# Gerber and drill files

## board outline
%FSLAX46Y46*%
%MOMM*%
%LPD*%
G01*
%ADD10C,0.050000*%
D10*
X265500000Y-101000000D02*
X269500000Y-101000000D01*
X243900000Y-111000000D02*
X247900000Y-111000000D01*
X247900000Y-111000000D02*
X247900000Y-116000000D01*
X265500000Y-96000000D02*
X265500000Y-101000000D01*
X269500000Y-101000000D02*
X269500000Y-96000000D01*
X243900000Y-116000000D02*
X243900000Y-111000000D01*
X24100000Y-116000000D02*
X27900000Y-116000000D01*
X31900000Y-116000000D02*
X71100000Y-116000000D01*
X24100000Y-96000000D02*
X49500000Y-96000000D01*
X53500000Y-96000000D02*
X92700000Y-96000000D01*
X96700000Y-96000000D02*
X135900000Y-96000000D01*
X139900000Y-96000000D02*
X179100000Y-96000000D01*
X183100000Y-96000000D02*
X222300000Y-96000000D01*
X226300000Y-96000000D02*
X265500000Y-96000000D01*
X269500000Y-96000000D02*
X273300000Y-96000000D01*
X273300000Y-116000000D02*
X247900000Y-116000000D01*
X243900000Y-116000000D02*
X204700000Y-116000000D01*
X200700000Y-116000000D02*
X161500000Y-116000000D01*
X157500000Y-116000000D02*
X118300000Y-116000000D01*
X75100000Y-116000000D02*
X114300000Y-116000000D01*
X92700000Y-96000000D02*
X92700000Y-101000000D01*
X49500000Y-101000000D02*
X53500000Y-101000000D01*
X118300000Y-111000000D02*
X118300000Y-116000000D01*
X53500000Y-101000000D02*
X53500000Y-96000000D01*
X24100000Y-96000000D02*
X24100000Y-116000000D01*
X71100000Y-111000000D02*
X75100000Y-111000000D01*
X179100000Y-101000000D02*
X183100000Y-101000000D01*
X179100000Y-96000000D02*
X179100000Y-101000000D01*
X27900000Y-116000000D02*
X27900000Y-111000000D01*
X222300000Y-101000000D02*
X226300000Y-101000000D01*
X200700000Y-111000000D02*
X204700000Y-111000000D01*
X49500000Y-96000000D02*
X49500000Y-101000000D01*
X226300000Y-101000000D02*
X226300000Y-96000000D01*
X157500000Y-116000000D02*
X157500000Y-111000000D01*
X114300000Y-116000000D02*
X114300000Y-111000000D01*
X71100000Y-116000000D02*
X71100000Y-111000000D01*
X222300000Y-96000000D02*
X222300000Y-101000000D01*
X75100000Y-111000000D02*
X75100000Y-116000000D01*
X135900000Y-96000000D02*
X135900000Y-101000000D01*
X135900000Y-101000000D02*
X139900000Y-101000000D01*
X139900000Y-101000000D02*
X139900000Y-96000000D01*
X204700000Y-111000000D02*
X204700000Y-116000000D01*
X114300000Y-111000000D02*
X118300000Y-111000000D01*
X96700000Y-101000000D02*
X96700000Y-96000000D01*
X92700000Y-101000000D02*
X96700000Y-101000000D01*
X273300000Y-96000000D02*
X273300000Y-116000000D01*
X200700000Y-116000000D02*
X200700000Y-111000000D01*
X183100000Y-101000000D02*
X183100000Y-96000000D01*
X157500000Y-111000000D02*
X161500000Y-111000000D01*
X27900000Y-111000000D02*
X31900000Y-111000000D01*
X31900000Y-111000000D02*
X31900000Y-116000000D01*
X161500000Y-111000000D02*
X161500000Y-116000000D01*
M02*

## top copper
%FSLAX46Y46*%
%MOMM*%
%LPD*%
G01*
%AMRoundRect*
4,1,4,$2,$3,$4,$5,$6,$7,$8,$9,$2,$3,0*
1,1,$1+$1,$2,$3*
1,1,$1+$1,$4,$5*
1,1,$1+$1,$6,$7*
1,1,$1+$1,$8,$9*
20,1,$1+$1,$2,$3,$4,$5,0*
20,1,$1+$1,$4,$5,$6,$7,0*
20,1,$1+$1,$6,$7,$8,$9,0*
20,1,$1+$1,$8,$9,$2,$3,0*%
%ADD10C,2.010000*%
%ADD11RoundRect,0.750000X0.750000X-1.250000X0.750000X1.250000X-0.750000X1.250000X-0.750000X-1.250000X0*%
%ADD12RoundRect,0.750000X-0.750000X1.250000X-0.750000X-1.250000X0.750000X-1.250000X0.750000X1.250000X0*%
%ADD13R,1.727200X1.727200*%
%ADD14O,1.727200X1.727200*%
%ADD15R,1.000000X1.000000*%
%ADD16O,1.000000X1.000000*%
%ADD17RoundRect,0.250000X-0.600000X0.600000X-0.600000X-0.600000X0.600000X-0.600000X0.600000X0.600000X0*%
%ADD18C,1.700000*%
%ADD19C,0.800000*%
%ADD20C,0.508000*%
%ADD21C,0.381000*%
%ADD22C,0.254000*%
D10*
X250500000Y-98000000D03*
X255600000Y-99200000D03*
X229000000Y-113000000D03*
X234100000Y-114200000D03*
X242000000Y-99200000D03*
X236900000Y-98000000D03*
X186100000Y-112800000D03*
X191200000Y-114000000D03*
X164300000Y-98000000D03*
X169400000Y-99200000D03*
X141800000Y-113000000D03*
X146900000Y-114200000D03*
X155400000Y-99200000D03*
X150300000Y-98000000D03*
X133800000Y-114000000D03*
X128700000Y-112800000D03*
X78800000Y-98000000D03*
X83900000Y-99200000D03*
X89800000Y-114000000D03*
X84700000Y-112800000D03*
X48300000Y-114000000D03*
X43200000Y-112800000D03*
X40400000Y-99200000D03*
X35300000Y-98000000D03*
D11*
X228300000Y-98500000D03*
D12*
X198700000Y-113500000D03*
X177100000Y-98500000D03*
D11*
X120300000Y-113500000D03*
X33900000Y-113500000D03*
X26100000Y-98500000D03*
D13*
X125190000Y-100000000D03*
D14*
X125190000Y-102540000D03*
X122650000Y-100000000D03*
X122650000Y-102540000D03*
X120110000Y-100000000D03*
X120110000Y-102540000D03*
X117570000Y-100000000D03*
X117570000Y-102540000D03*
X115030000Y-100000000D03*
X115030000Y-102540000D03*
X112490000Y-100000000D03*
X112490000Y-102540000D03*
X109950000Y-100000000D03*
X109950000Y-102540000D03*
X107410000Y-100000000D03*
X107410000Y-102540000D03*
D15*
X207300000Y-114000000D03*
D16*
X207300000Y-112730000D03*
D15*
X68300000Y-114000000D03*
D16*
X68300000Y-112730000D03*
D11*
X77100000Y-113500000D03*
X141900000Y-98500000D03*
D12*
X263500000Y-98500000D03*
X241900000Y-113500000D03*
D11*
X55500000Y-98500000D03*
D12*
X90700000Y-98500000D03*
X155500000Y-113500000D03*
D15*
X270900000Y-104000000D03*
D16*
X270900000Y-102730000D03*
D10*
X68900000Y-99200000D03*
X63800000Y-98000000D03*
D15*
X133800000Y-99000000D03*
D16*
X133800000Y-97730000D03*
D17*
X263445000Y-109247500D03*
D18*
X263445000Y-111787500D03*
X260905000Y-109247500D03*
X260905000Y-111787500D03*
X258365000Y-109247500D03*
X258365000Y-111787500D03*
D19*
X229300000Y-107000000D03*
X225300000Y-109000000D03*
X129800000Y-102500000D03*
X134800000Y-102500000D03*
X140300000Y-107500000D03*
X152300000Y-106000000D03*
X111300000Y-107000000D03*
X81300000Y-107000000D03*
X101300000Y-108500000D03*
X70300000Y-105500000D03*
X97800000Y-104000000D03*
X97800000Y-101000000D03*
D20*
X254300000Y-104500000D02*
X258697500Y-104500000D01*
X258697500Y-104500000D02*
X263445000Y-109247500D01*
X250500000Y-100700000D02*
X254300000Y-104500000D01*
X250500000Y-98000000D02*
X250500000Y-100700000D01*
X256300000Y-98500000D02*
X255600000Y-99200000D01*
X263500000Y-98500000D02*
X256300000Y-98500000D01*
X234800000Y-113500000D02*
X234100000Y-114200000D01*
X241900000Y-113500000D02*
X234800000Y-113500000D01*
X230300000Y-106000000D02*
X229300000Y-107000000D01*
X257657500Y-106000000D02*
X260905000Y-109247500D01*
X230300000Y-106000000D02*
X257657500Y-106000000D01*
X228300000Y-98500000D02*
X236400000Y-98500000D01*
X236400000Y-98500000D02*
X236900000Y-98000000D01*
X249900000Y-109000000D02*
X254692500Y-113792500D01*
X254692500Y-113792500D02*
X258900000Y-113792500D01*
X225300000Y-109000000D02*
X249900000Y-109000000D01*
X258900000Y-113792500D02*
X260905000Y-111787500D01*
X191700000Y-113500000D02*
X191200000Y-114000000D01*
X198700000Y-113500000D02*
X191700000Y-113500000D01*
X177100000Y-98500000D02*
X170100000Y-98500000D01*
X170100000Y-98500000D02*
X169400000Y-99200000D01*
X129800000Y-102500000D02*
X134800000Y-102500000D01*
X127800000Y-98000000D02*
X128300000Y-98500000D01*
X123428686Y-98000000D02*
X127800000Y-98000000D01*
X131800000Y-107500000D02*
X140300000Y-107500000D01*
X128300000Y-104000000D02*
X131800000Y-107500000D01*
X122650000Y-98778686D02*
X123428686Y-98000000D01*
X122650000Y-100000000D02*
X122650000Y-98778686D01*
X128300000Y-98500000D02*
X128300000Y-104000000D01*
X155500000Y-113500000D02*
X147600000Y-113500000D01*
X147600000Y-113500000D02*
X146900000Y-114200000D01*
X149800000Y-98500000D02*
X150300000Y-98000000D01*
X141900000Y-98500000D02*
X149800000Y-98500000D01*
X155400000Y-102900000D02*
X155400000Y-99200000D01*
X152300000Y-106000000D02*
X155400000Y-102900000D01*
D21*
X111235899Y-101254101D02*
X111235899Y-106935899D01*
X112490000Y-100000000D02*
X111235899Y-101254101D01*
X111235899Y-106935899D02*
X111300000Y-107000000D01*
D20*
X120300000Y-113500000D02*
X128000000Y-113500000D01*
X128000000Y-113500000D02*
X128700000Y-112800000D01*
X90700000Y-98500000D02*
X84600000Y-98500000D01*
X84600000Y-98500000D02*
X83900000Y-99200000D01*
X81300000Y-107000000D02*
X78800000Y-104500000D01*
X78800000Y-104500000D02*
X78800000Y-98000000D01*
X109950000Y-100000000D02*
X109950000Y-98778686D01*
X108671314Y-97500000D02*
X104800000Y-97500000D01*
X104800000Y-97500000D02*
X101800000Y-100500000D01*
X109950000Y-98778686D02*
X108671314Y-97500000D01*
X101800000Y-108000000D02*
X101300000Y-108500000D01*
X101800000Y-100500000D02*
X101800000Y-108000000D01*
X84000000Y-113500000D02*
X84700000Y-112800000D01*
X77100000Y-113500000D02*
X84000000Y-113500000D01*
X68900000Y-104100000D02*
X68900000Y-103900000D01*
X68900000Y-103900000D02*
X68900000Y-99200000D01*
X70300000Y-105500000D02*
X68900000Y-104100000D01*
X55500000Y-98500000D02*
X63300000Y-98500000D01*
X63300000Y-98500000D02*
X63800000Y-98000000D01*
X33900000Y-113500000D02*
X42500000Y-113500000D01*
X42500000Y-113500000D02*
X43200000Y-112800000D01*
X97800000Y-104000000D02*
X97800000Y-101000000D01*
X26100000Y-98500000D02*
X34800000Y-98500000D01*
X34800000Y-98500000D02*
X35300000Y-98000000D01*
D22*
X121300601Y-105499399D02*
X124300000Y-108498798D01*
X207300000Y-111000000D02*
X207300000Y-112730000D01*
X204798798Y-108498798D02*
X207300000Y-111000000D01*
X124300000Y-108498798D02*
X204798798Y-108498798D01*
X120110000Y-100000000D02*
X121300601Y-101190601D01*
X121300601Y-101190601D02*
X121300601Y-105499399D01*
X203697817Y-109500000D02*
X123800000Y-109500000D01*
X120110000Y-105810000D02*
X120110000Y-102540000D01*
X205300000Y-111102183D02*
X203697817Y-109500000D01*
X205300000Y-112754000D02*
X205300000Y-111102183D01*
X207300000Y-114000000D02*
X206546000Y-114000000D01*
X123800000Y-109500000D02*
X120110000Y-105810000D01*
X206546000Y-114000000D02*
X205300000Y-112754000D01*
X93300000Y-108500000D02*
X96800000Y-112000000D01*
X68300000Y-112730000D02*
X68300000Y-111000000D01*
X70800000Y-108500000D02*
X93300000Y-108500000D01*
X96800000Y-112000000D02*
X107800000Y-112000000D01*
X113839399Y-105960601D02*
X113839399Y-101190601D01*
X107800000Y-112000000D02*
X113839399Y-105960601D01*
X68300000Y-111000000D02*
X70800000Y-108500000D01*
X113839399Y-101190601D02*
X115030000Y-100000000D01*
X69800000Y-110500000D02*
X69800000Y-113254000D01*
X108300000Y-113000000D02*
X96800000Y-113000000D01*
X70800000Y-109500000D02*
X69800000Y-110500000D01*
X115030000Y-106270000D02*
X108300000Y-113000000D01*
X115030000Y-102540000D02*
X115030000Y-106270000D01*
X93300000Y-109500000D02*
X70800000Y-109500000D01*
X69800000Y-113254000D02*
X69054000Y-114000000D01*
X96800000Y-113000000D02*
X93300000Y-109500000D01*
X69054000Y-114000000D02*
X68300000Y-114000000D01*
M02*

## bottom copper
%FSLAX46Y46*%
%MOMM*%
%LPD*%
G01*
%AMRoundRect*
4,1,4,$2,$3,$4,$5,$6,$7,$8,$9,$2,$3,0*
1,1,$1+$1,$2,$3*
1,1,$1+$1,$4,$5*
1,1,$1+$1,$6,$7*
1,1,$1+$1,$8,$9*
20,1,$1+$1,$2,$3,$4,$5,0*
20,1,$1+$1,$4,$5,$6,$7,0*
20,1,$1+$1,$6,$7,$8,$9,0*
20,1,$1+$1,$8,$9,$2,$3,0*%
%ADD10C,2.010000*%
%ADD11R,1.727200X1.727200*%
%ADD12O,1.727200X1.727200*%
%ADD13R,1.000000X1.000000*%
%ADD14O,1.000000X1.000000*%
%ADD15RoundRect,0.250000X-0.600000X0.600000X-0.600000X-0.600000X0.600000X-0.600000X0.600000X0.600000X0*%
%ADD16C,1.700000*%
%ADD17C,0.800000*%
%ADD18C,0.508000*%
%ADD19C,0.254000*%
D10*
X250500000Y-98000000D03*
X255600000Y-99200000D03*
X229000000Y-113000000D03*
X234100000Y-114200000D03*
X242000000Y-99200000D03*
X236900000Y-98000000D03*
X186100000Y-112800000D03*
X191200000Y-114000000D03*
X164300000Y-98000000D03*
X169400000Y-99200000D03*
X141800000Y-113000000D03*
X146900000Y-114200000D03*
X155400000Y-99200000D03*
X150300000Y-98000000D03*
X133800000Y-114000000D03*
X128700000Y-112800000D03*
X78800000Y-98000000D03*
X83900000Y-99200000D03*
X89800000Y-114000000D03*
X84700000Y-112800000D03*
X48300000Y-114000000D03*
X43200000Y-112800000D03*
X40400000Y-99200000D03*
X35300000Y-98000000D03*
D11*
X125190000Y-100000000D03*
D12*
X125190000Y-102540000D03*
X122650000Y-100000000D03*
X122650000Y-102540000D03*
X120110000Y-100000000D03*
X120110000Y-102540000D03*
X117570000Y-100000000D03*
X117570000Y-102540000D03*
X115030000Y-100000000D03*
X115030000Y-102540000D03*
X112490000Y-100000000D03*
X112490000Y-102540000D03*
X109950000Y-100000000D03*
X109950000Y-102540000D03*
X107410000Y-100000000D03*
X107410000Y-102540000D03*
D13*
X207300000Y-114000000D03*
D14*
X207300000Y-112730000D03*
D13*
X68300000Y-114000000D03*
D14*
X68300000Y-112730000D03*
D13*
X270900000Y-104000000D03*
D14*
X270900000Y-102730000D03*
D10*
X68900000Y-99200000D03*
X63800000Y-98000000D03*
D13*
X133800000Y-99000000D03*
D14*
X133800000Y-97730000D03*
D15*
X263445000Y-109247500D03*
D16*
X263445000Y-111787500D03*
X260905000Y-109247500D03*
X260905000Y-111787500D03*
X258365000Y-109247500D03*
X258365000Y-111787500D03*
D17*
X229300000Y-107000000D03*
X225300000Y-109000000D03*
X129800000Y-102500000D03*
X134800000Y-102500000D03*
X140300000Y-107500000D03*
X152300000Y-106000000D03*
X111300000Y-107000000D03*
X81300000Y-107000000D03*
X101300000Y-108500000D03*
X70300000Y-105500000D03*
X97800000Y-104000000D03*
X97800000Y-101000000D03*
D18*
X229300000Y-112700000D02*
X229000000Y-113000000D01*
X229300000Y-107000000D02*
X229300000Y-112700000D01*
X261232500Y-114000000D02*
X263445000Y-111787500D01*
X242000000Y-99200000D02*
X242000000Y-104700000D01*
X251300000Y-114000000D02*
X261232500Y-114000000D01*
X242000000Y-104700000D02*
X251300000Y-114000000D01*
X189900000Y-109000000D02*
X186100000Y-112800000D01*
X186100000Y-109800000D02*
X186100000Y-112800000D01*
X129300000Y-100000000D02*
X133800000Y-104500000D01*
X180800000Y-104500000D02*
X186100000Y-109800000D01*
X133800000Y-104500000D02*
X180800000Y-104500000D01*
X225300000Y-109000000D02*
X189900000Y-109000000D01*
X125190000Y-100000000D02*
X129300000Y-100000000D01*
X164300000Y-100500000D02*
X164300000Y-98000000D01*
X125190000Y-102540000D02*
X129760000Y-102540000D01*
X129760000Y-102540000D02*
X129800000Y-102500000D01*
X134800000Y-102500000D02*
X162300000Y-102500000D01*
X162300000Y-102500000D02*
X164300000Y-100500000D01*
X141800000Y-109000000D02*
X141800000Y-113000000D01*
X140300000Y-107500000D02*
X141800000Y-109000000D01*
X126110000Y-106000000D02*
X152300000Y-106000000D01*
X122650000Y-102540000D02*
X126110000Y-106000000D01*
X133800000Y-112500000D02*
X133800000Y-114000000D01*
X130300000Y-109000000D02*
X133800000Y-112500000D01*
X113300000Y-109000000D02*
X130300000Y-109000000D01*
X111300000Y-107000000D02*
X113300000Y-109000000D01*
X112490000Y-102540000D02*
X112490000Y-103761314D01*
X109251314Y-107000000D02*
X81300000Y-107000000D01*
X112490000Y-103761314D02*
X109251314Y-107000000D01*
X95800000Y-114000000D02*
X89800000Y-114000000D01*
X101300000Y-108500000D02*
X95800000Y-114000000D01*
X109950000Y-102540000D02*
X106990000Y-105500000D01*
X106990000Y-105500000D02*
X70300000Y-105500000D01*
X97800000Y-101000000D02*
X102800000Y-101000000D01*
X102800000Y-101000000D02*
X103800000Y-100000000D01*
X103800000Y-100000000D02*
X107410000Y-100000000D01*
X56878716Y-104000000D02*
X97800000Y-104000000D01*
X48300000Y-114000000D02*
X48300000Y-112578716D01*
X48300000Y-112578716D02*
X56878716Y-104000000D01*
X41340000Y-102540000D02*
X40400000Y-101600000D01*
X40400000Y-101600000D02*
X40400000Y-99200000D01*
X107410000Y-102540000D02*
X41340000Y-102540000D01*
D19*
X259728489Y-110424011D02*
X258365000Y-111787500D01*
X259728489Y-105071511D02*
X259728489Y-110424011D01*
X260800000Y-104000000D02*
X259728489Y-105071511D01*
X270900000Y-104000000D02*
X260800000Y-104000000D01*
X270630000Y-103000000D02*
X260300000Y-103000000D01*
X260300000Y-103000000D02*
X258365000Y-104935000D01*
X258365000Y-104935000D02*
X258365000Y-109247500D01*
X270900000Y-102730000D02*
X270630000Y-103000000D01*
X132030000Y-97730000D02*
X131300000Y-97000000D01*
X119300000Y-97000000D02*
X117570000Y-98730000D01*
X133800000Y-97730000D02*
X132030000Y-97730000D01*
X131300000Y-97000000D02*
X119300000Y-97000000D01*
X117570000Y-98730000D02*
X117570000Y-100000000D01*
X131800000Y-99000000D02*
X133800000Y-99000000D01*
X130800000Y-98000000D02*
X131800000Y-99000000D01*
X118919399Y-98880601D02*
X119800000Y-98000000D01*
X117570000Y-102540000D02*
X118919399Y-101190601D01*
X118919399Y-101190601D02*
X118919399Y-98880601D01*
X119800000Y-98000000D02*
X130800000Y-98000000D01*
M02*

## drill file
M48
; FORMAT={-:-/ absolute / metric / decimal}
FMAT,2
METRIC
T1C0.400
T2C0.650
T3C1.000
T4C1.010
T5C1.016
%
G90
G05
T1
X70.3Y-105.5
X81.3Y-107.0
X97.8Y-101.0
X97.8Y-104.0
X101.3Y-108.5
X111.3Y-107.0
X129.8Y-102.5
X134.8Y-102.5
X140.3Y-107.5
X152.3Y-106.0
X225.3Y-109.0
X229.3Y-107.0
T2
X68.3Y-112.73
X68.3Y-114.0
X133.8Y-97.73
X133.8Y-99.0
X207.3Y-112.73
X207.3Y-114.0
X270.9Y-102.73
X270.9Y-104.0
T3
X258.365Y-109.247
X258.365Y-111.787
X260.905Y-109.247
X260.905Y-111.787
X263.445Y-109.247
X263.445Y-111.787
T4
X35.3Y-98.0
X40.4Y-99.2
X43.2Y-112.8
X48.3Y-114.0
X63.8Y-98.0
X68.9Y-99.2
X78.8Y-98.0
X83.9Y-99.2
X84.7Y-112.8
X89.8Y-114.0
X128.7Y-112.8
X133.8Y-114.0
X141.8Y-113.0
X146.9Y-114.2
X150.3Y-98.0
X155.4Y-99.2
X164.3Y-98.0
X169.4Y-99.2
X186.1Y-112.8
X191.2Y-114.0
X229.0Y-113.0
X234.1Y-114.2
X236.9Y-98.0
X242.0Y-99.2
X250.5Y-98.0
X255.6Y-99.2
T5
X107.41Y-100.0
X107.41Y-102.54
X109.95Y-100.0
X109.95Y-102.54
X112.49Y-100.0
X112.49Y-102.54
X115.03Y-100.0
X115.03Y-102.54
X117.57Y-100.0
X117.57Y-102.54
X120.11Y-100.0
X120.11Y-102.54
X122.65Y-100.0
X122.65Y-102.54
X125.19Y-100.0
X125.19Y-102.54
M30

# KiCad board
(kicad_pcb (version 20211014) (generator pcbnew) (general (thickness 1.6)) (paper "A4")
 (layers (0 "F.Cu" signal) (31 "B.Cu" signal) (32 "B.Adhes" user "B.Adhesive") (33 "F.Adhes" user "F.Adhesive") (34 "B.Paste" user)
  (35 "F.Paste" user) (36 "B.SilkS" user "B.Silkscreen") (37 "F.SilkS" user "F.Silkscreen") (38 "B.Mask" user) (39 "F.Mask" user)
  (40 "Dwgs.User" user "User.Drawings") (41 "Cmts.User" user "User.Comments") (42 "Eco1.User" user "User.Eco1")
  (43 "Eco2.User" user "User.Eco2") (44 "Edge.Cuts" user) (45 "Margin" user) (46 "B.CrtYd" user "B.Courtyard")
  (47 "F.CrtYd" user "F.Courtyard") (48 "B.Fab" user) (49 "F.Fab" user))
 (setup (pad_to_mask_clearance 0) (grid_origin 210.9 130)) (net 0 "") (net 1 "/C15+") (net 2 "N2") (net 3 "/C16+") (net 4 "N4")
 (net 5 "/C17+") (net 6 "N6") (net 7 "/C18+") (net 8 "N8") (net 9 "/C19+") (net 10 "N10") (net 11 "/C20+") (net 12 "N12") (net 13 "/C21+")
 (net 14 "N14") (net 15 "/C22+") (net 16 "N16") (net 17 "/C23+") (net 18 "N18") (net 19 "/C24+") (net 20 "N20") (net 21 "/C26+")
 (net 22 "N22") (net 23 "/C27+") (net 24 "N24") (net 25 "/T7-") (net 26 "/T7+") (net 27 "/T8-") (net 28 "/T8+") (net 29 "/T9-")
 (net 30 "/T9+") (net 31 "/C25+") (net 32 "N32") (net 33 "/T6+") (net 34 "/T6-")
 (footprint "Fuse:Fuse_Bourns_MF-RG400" (layer "F.Cu") (at 250.5 98)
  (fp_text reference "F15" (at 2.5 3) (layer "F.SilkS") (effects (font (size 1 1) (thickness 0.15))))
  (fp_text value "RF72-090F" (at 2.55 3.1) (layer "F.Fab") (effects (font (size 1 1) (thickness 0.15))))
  (pad "1" thru_hole circle locked (at 0 0) (size 2.01 2.01) (drill 1.01) (layers *.Cu *.Mask) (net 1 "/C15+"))
  (pad "2" thru_hole circle locked (at 5.1 1.2) (size 2.01 2.01) (drill 1.01) (layers *.Cu *.Mask) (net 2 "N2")))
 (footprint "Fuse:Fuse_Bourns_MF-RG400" (layer "F.Cu") (at 229 113)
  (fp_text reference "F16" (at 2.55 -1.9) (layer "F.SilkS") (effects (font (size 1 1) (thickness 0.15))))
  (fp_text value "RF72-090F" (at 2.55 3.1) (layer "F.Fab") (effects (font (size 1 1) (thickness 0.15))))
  (pad "1" thru_hole circle locked (at 0 0) (size 2.01 2.01) (drill 1.01) (layers *.Cu *.Mask) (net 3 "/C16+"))
  (pad "2" thru_hole circle locked (at 5.1 1.2) (size 2.01 2.01) (drill 1.01) (layers *.Cu *.Mask) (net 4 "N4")))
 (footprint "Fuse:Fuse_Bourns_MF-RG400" (layer "F.Cu") (at 242 99.2 180)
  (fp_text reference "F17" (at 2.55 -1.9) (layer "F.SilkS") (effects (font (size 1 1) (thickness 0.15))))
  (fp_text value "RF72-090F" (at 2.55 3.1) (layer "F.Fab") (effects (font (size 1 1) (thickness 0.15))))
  (pad "1" thru_hole circle locked (at 0 0 180) (size 2.01 2.01) (drill 1.01) (layers *.Cu *.Mask) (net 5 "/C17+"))
  (pad "2" thru_hole circle locked (at 5.1 1.2 180) (size 2.01 2.01) (drill 1.01) (layers *.Cu *.Mask) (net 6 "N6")))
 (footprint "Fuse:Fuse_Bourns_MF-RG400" (layer "F.Cu") (at 186.1 112.8)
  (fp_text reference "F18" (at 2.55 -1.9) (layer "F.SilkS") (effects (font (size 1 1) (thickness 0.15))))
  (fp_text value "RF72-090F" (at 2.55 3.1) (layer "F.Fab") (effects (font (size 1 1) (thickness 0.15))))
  (pad "1" thru_hole circle locked (at 0 0) (size 2.01 2.01) (drill 1.01) (layers *.Cu *.Mask) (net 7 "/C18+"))
  (pad "2" thru_hole circle locked (at 5.1 1.2) (size 2.01 2.01) (drill 1.01) (layers *.Cu *.Mask) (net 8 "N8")))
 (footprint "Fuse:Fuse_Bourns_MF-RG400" (layer "F.Cu") (at 164.3 98)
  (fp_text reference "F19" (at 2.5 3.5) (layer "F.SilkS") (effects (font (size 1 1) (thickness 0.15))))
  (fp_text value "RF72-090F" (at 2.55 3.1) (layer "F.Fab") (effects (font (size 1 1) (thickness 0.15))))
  (pad "1" thru_hole circle locked (at 0 0) (size 2.01 2.01) (drill 1.01) (layers *.Cu *.Mask) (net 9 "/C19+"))
  (pad "2" thru_hole circle locked (at 5.1 1.2) (size 2.01 2.01) (drill 1.01) (layers *.Cu *.Mask) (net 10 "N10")))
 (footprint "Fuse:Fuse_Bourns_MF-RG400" (layer "F.Cu") (at 141.8 113)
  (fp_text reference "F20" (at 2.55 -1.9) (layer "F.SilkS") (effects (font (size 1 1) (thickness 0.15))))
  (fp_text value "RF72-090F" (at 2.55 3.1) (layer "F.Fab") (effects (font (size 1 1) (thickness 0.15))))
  (pad "1" thru_hole circle locked (at 0 0) (size 2.01 2.01) (drill 1.01) (layers *.Cu *.Mask) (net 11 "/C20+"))
  (pad "2" thru_hole circle locked (at 5.1 1.2) (size 2.01 2.01) (drill 1.01) (layers *.Cu *.Mask) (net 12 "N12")))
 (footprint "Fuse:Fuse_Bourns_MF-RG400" (layer "F.Cu") (at 155.4 99.2 180)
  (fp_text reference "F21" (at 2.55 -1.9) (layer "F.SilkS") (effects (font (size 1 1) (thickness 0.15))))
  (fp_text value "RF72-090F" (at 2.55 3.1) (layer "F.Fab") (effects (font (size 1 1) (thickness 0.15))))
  (pad "1" thru_hole circle locked (at 0 0 180) (size 2.01 2.01) (drill 1.01) (layers *.Cu *.Mask) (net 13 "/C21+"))
  (pad "2" thru_hole circle locked (at 5.1 1.2 180) (size 2.01 2.01) (drill 1.01) (layers *.Cu *.Mask) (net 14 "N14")))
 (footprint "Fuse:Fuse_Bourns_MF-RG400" (layer "F.Cu") (at 133.8 114 180)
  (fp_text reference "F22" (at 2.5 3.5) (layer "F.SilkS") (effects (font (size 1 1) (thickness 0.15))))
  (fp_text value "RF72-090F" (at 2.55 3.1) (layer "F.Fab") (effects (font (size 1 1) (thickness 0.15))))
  (pad "1" thru_hole circle locked (at 0 0 180) (size 2.01 2.01) (drill 1.01) (layers *.Cu *.Mask) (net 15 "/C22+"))
  (pad "2" thru_hole circle locked (at 5.1 1.2 180) (size 2.01 2.01) (drill 1.01) (layers *.Cu *.Mask) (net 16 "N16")))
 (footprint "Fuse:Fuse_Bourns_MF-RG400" (layer "F.Cu") (at 78.8 98)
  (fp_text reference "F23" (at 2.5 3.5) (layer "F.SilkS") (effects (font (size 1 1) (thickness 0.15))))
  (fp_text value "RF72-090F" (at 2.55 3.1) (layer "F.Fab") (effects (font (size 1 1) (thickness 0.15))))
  (pad "1" thru_hole circle locked (at 0 0) (size 2.01 2.01) (drill 1.01) (layers *.Cu *.Mask) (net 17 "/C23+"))
  (pad "2" thru_hole circle locked (at 5.1 1.2) (size 2.01 2.01) (drill 1.01) (layers *.Cu *.Mask) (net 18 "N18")))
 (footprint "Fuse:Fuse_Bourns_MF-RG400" (layer "F.Cu") (at 89.8 114 180)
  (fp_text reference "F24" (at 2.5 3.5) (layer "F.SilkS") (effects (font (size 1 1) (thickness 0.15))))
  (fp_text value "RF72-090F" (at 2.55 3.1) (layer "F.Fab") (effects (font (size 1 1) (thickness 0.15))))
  (pad "1" thru_hole circle locked (at 0 0 180) (size 2.01 2.01) (drill 1.01) (layers *.Cu *.Mask) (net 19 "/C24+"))
  (pad "2" thru_hole circle locked (at 5.1 1.2 180) (size 2.01 2.01) (drill 1.01) (layers *.Cu *.Mask) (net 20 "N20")))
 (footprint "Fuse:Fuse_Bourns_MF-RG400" (layer "F.Cu") (at 48.3 114 180)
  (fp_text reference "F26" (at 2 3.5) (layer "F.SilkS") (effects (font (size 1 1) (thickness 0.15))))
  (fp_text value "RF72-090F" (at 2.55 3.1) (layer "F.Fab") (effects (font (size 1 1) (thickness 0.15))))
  (pad "1" thru_hole circle locked (at 0 0 180) (size 2.01 2.01) (drill 1.01) (layers *.Cu *.Mask) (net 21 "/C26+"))
  (pad "2" thru_hole circle locked (at 5.1 1.2 180) (size 2.01 2.01) (drill 1.01) (layers *.Cu *.Mask) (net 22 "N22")))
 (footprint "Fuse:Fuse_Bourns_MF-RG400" (layer "F.Cu") (at 40.4 99.2 180)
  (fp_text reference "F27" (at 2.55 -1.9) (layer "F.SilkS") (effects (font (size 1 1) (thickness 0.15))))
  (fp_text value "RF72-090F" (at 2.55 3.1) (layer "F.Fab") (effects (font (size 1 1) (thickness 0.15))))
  (pad "1" thru_hole circle locked (at 0 0 180) (size 2.01 2.01) (drill 1.01) (layers *.Cu *.Mask) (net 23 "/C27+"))
  (pad "2" thru_hole circle locked (at 5.1 1.2 180) (size 2.01 2.01) (drill 1.01) (layers *.Cu *.Mask) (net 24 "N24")))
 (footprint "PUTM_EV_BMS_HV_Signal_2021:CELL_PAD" (layer "F.Cu") (at 228.3 98.5 90)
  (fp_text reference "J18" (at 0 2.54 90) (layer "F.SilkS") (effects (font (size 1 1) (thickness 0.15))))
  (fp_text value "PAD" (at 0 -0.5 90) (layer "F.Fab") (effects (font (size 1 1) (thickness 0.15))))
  (pad "1" smd roundrect locked (at 0 0 90) (size 4 3) (layers "F.Cu" "F.Paste" "F.Mask") (roundrect_rratio 0.25) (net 6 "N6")))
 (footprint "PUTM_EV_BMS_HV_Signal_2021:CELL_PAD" (layer "F.Cu") (at 198.7 113.5 -90)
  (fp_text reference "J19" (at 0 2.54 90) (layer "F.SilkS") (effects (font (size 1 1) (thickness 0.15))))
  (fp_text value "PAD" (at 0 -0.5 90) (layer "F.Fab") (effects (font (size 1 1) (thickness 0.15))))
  (pad "1" smd roundrect locked (at 0 0 270) (size 4 3) (layers "F.Cu" "F.Paste" "F.Mask") (roundrect_rratio 0.25) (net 8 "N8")))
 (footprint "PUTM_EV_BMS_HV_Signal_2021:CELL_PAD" (layer "F.Cu") (at 177.1 98.5 -90)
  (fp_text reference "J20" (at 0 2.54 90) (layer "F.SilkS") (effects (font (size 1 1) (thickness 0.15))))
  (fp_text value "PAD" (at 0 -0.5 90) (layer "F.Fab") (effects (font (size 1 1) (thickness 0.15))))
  (pad "1" smd roundrect locked (at 0 0 270) (size 4 3) (layers "F.Cu" "F.Paste" "F.Mask") (roundrect_rratio 0.25) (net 10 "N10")))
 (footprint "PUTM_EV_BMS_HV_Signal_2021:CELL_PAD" (layer "F.Cu") (at 120.3 113.5 90)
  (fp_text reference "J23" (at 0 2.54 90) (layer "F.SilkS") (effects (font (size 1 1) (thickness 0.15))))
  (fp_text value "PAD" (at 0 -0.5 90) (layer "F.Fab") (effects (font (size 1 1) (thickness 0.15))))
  (pad "1" smd roundrect locked (at 0 0 90) (size 4 3) (layers "F.Cu" "F.Paste" "F.Mask") (roundrect_rratio 0.25) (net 16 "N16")))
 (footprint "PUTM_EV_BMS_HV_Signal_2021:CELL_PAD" (layer "F.Cu") (at 33.9 113.5 90)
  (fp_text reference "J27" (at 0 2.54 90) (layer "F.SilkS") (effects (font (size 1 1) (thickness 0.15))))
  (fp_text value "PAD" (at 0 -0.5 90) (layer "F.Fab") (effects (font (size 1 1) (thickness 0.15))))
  (pad "1" smd roundrect locked (at 0 0 90) (size 4 3) (layers "F.Cu" "F.Paste" "F.Mask") (roundrect_rratio 0.25) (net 22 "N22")))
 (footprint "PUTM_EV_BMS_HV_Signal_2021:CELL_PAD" (layer "F.Cu") (at 26.1 98.5 90)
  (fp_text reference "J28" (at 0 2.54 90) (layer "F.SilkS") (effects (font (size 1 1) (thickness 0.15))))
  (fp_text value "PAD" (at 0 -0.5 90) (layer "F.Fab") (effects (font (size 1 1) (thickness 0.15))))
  (pad "1" smd roundrect locked (at 0 0 90) (size 4 3) (layers "F.Cu" "F.Paste" "F.Mask") (roundrect_rratio 0.25) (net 24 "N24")))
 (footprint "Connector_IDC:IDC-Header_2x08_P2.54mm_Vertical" (layer "F.Cu") (at 125.19 100 -90)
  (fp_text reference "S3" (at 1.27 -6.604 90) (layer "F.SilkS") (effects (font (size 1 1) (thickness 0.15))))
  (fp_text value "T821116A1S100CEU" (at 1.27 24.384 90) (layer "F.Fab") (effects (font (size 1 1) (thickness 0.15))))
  (pad "1" thru_hole rect locked (at 0 0 270) (size 1.7272 1.7272) (drill 1.016) (layers *.Cu *.Mask) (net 7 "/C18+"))
  (pad "2" thru_hole oval locked (at 2.54 0 270) (size 1.7272 1.7272) (drill 1.016) (layers *.Cu *.Mask) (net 9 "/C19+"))
  (pad "3" thru_hole oval locked (at 0 2.54 270) (size 1.7272 1.7272) (drill 1.016) (layers *.Cu *.Mask) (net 11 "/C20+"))
  (pad "4" thru_hole oval locked (at 2.54 2.54 270) (size 1.7272 1.7272) (drill 1.016) (layers *.Cu *.Mask) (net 13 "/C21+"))
  (pad "5" thru_hole oval locked (at 0 5.08 270) (size 1.7272 1.7272) (drill 1.016) (layers *.Cu *.Mask) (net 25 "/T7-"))
  (pad "6" thru_hole oval locked (at 2.54 5.08 270) (size 1.7272 1.7272) (drill 1.016) (layers *.Cu *.Mask) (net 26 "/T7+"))
  (pad "7" thru_hole oval locked (at 0 7.62 270) (size 1.7272 1.7272) (drill 1.016) (layers *.Cu *.Mask) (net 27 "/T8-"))
  (pad "8" thru_hole oval locked (at 2.54 7.62 270) (size 1.7272 1.7272) (drill 1.016) (layers *.Cu *.Mask) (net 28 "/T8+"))
  (pad "9" thru_hole oval locked (at 0 10.16 270) (size 1.7272 1.7272) (drill 1.016) (layers *.Cu *.Mask) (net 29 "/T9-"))
  (pad "10" thru_hole oval locked (at 2.54 10.16 270) (size 1.7272 1.7272) (drill 1.016) (layers *.Cu *.Mask) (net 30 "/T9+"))
  (pad "11" thru_hole oval locked (at 0 12.7 270) (size 1.7272 1.7272) (drill 1.016) (layers *.Cu *.Mask) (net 15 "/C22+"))
  (pad "12" thru_hole oval locked (at 2.54 12.7 270) (size 1.7272 1.7272) (drill 1.016) (layers *.Cu *.Mask) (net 17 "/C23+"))
  (pad "13" thru_hole oval locked (at 0 15.24 270) (size 1.7272 1.7272) (drill 1.016) (layers *.Cu *.Mask) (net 19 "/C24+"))
  (pad "14" thru_hole oval locked (at 2.54 15.24 270) (size 1.7272 1.7272) (drill 1.016) (layers *.Cu *.Mask) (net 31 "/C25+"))
  (pad "15" thru_hole oval locked (at 0 17.78 270) (size 1.7272 1.7272) (drill 1.016) (layers *.Cu *.Mask) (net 21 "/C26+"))
  (pad "16" thru_hole oval locked (at 2.54 17.78 270) (size 1.7272 1.7272) (drill 1.016) (layers *.Cu *.Mask) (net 23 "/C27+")))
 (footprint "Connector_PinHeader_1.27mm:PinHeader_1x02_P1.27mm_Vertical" (layer "F.Cu") (at 207.3 114 180)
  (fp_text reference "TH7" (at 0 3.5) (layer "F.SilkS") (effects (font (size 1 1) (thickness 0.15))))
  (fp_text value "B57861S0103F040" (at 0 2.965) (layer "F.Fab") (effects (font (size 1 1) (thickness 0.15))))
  (pad "1" thru_hole rect locked (at 0 0 180) (size 1 1) (drill 0.65) (layers *.Cu *.Mask) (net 26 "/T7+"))
  (pad "2" thru_hole oval locked (at 0 1.27 180) (size 1 1) (drill 0.65) (layers *.Cu *.Mask) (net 25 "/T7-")))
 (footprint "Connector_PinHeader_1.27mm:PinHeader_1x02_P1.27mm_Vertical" (layer "F.Cu") (at 68.3 114 180)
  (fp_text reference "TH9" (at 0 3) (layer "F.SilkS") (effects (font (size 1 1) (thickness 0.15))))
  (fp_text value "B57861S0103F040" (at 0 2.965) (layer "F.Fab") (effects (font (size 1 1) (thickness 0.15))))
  (pad "1" thru_hole rect locked (at 0 0 180) (size 1 1) (drill 0.65) (layers *.Cu *.Mask) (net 30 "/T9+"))
  (pad "2" thru_hole oval locked (at 0 1.27 180) (size 1 1) (drill 0.65) (layers *.Cu *.Mask) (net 29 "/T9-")))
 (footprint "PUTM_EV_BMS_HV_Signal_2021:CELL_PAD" (layer "F.Cu") (at 77.1 113.5 90)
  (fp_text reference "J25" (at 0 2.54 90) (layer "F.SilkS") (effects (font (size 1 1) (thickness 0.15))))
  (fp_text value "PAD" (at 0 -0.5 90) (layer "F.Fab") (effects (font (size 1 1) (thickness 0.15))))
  (pad "1" smd roundrect locked (at 0 0 90) (size 4 3) (layers "F.Cu" "F.Paste" "F.Mask") (roundrect_rratio 0.25) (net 20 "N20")))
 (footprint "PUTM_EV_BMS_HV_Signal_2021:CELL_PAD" (layer "F.Cu") (at 141.9 98.5 90)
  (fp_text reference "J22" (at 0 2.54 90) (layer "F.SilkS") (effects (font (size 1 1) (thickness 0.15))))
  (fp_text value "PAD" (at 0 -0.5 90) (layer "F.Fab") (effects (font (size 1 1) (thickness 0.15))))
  (pad "1" smd roundrect locked (at 0 0 90) (size 4 3) (layers "F.Cu" "F.Paste" "F.Mask") (roundrect_rratio 0.25) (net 14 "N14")))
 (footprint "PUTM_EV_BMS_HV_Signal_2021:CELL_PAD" (layer "F.Cu") (at 263.5 98.5 -90)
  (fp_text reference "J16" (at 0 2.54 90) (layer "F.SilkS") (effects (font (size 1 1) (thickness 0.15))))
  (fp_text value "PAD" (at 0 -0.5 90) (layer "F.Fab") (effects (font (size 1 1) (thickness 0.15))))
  (pad "1" smd roundrect locked (at 0 0 270) (size 4 3) (layers "F.Cu" "F.Paste" "F.Mask") (roundrect_rratio 0.25) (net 2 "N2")))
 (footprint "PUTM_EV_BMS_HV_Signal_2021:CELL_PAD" (layer "F.Cu") (at 241.9 113.5 -90)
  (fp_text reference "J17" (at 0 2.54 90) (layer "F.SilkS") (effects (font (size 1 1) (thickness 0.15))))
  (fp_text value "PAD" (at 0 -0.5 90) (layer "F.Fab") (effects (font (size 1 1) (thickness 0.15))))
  (pad "1" smd roundrect locked (at 0 0 270) (size 4 3) (layers "F.Cu" "F.Paste" "F.Mask") (roundrect_rratio 0.25) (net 4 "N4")))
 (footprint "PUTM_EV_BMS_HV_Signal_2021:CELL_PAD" (layer "F.Cu") (at 55.5 98.5 90)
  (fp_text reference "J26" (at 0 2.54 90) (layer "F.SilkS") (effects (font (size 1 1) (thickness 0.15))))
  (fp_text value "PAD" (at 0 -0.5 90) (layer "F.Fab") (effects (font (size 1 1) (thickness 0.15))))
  (pad "1" smd roundrect locked (at 0 0 90) (size 4 3) (layers "F.Cu" "F.Paste" "F.Mask") (roundrect_rratio 0.25) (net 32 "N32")))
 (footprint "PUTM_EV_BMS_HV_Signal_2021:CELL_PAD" (layer "F.Cu") (at 90.7 98.5 -90)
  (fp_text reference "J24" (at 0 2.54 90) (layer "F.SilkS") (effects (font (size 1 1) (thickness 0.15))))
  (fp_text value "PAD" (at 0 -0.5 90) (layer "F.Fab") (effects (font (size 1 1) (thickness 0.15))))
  (pad "1" smd roundrect locked (at 0 0 270) (size 4 3) (layers "F.Cu" "F.Paste" "F.Mask") (roundrect_rratio 0.25) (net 18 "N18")))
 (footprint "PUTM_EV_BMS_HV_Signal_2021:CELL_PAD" (layer "F.Cu") (at 155.5 113.5 -90)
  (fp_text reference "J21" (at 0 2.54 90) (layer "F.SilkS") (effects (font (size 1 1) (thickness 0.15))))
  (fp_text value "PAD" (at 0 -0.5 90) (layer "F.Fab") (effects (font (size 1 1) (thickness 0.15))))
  (pad "1" smd roundrect locked (at 0 0 270) (size 4 3) (layers "F.Cu" "F.Paste" "F.Mask") (roundrect_rratio 0.25) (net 12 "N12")))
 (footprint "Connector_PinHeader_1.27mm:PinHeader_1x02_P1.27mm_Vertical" (layer "F.Cu") (at 270.9 104 180)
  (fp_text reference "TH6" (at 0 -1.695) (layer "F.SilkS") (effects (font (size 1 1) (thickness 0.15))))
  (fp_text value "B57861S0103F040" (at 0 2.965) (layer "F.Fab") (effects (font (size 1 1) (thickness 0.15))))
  (pad "1" thru_hole rect locked (at 0 0 180) (size 1 1) (drill 0.65) (layers *.Cu *.Mask) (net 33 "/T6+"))
  (pad "2" thru_hole oval locked (at 0 1.27 180) (size 1 1) (drill 0.65) (layers *.Cu *.Mask) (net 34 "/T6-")))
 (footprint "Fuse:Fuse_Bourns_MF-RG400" (layer "F.Cu") (at 68.9 99.2 180)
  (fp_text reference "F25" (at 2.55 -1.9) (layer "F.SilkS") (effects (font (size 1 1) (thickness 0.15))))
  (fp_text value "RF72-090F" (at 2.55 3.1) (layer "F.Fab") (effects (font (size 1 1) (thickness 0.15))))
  (pad "1" thru_hole circle locked (at 0 0 180) (size 2.01 2.01) (drill 1.01) (layers *.Cu *.Mask) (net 31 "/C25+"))
  (pad "2" thru_hole circle locked (at 5.1 1.2 180) (size 2.01 2.01) (drill 1.01) (layers *.Cu *.Mask) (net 32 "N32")))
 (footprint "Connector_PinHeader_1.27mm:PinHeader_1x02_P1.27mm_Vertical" (layer "F.Cu") (at 133.8 99 180)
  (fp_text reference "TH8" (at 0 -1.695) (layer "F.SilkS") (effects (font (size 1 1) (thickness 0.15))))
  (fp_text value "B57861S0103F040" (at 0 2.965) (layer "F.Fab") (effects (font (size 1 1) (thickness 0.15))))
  (pad "1" thru_hole rect locked (at 0 0 180) (size 1 1) (drill 0.65) (layers *.Cu *.Mask) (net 28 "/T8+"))
  (pad "2" thru_hole oval locked (at 0 1.27 180) (size 1 1) (drill 0.65) (layers *.Cu *.Mask) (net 27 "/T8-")))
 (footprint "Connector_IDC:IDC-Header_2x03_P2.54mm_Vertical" (layer "F.Cu") (at 263.445 109.2475 -90)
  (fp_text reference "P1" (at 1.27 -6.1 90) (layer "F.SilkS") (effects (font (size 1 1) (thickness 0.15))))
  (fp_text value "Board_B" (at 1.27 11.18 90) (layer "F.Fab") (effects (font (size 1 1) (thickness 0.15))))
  (pad "1" thru_hole roundrect locked (at 0 0 270) (size 1.7 1.7) (drill 1) (layers *.Cu *.Mask) (roundrect_rratio 0.1470588235)
   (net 1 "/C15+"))
  (pad "2" thru_hole circle locked (at 2.54 0 270) (size 1.7 1.7) (drill 1) (layers *.Cu *.Mask) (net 5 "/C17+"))
  (pad "3" thru_hole circle locked (at 0 2.54 270) (size 1.7 1.7) (drill 1) (layers *.Cu *.Mask) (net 3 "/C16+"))
  (pad "4" thru_hole circle locked (at 2.54 2.54 270) (size 1.7 1.7) (drill 1) (layers *.Cu *.Mask) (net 7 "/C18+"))
  (pad "5" thru_hole circle locked (at 0 5.08 270) (size 1.7 1.7) (drill 1) (layers *.Cu *.Mask) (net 34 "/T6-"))
  (pad "6" thru_hole circle locked (at 2.54 5.08 270) (size 1.7 1.7) (drill 1) (layers *.Cu *.Mask) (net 33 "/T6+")))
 (gr_line (start 265.5 101) (end 269.5 101) (layer "Edge.Cuts") (width 0.05))
 (gr_line (start 243.9 111) (end 247.9 111) (layer "Edge.Cuts") (width 0.05))
 (gr_line (start 247.9 111) (end 247.9 116) (layer "Edge.Cuts") (width 0.05))
 (gr_line (start 265.5 96) (end 265.5 101) (layer "Edge.Cuts") (width 0.05))
 (gr_line (start 269.5 101) (end 269.5 96) (layer "Edge.Cuts") (width 0.05))
 (gr_line (start 243.9 116) (end 243.9 111) (layer "Edge.Cuts") (width 0.05))
 (gr_line (start 24.1 116) (end 27.9 116) (layer "Edge.Cuts") (width 0.05))
 (gr_line (start 31.9 116) (end 71.1 116) (layer "Edge.Cuts") (width 0.05))
 (gr_line (start 24.1 96) (end 49.5 96) (layer "Edge.Cuts") (width 0.05))
 (gr_line (start 53.5 96) (end 92.7 96) (layer "Edge.Cuts") (width 0.05))
 (gr_line (start 96.7 96) (end 135.9 96) (layer "Edge.Cuts") (width 0.05))
 (gr_line (start 139.9 96) (end 179.1 96) (layer "Edge.Cuts") (width 0.05))
 (gr_line (start 183.1 96) (end 222.3 96) (layer "Edge.Cuts") (width 0.05))
 (gr_line (start 226.3 96) (end 265.5 96) (layer "Edge.Cuts") (width 0.05))
 (gr_line (start 269.5 96) (end 273.3 96) (layer "Edge.Cuts") (width 0.05))
 (gr_line (start 273.3 116) (end 247.9 116) (layer "Edge.Cuts") (width 0.05))
 (gr_line (start 243.9 116) (end 204.7 116) (layer "Edge.Cuts") (width 0.05))
 (gr_line (start 200.7 116) (end 161.5 116) (layer "Edge.Cuts") (width 0.05))
 (gr_line (start 157.5 116) (end 118.3 116) (layer "Edge.Cuts") (width 0.05))
 (gr_line (start 75.1 116) (end 114.3 116) (layer "Edge.Cuts") (width 0.05))
 (gr_line (start 92.7 96) (end 92.7 101) (layer "Edge.Cuts") (width 0.05))
 (gr_line (start 49.5 101) (end 53.5 101) (layer "Edge.Cuts") (width 0.05))
 (gr_line (start 118.3 111) (end 118.3 116) (layer "Edge.Cuts") (width 0.05))
 (gr_line (start 53.5 101) (end 53.5 96) (layer "Edge.Cuts") (width 0.05))
 (gr_line (start 24.1 96) (end 24.1 116) (layer "Edge.Cuts") (width 0.05))
 (gr_line (start 71.1 111) (end 75.1 111) (layer "Edge.Cuts") (width 0.05))
 (gr_line (start 179.1 101) (end 183.1 101) (layer "Edge.Cuts") (width 0.05))
 (gr_line (start 179.1 96) (end 179.1 101) (layer "Edge.Cuts") (width 0.05))
 (gr_line (start 27.9 116) (end 27.9 111) (layer "Edge.Cuts") (width 0.05))
 (gr_line (start 222.3 101) (end 226.3 101) (layer "Edge.Cuts") (width 0.05))
 (gr_line (start 200.7 111) (end 204.7 111) (layer "Edge.Cuts") (width 0.05))
 (gr_line (start 49.5 96) (end 49.5 101) (layer "Edge.Cuts") (width 0.05))
 (gr_line (start 226.3 101) (end 226.3 96) (layer "Edge.Cuts") (width 0.05))
 (gr_line (start 157.5 116) (end 157.5 111) (layer "Edge.Cuts") (width 0.05))
 (gr_line (start 114.3 116) (end 114.3 111) (layer "Edge.Cuts") (width 0.05))
 (gr_line (start 71.1 116) (end 71.1 111) (layer "Edge.Cuts") (width 0.05))
 (gr_line (start 222.3 96) (end 222.3 101) (layer "Edge.Cuts") (width 0.05))
 (gr_line (start 75.1 111) (end 75.1 116) (layer "Edge.Cuts") (width 0.05))
 (gr_line (start 135.9 96) (end 135.9 101) (layer "Edge.Cuts") (width 0.05))
 (gr_line (start 135.9 101) (end 139.9 101) (layer "Edge.Cuts") (width 0.05))
 (gr_line (start 139.9 101) (end 139.9 96) (layer "Edge.Cuts") (width 0.05))
 (gr_line (start 204.7 111) (end 204.7 116) (layer "Edge.Cuts") (width 0.05))
 (gr_line (start 114.3 111) (end 118.3 111) (layer "Edge.Cuts") (width 0.05))
 (gr_line (start 96.7 101) (end 96.7 96) (layer "Edge.Cuts") (width 0.05))
 (gr_line (start 92.7 101) (end 96.7 101) (layer "Edge.Cuts") (width 0.05))
 (gr_line (start 273.3 96) (end 273.3 116) (layer "Edge.Cuts") (width 0.05))
 (gr_line (start 200.7 116) (end 200.7 111) (layer "Edge.Cuts") (width 0.05))
 (gr_line (start 183.1 101) (end 183.1 96) (layer "Edge.Cuts") (width 0.05))
 (gr_line (start 157.5 111) (end 161.5 111) (layer "Edge.Cuts") (width 0.05))
 (gr_line (start 27.9 111) (end 31.9 111) (layer "Edge.Cuts") (width 0.05))
 (gr_line (start 31.9 111) (end 31.9 116) (layer "Edge.Cuts") (width 0.05))
 (gr_line (start 161.5 111) (end 161.5 116) (layer "Edge.Cuts") (width 0.05))
 (segment (start 254.3 104.5) (end 258.6975 104.5) (width 0.508) (layer "F.Cu") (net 1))
 (segment (start 258.6975 104.5) (end 263.445 109.2475) (width 0.508) (layer "F.Cu") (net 1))
 (segment (start 250.5 100.7) (end 254.3 104.5) (width 0.508) (layer "F.Cu") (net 1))
 (segment (start 250.5 98) (end 250.5 100.7) (width 0.508) (layer "F.Cu") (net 1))
 (segment (start 256.3 98.5) (end 255.6 99.2) (width 0.508) (layer "F.Cu") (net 2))
 (segment (start 263.5 98.5) (end 256.3 98.5) (width 0.508) (layer "F.Cu") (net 2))
 (segment (start 234.8 113.5) (end 234.1 114.2) (width 0.508) (layer "F.Cu") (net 4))
 (segment (start 241.9 113.5) (end 234.8 113.5) (width 0.508) (layer "F.Cu") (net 4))
 (segment (start 230.3 106) (end 229.3 107) (width 0.508) (layer "F.Cu") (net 3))
 (segment (start 257.6575 106) (end 260.905 109.2475) (width 0.508) (layer "F.Cu") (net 3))
 (segment (start 230.3 106) (end 257.6575 106) (width 0.508) (layer "F.Cu") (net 3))
 (via (at 229.3 107) (size 0.8) (drill 0.4) (layers "F.Cu" "B.Cu") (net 3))
 (segment (start 229.3 112.7) (end 229 113) (width 0.508) (layer "B.Cu") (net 3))
 (segment (start 229.3 107) (end 229.3 112.7) (width 0.508) (layer "B.Cu") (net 3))
 (segment (start 228.3 98.5) (end 236.4 98.5) (width 0.508) (layer "F.Cu") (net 6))
 (segment (start 236.4 98.5) (end 236.9 98) (width 0.508) (layer "F.Cu") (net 6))
 (segment (start 261.2325 114) (end 263.445 111.7875) (width 0.508) (layer "B.Cu") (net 5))
 (segment (start 242 99.2) (end 242 104.7) (width 0.508) (layer "B.Cu") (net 5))
 (segment (start 251.3 114) (end 261.2325 114) (width 0.508) (layer "B.Cu") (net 5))
 (segment (start 242 104.7) (end 251.3 114) (width 0.508) (layer "B.Cu") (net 5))
 (segment (start 249.9 109) (end 254.6925 113.7925) (width 0.508) (layer "F.Cu") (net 7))
 (segment (start 254.6925 113.7925) (end 258.9 113.7925) (width 0.508) (layer "F.Cu") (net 7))
 (segment (start 225.3 109) (end 249.9 109) (width 0.508) (layer "F.Cu") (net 7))
 (segment (start 258.9 113.7925) (end 260.905 111.7875) (width 0.508) (layer "F.Cu") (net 7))
 (via (at 225.3 109) (size 0.8) (drill 0.4) (layers "F.Cu" "B.Cu") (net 7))
 (segment (start 189.9 109) (end 186.1 112.8) (width 0.508) (layer "B.Cu") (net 7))
 (segment (start 186.1 109.8) (end 186.1 112.8) (width 0.508) (layer "B.Cu") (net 7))
 (segment (start 129.3 100) (end 133.8 104.5) (width 0.508) (layer "B.Cu") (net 7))
 (segment (start 180.8 104.5) (end 186.1 109.8) (width 0.508) (layer "B.Cu") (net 7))
 (segment (start 133.8 104.5) (end 180.8 104.5) (width 0.508) (layer "B.Cu") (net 7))
 (segment (start 225.3 109) (end 189.9 109) (width 0.508) (layer "B.Cu") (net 7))
 (segment (start 125.19 100) (end 129.3 100) (width 0.508) (layer "B.Cu") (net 7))
 (segment (start 191.7 113.5) (end 191.2 114) (width 0.508) (layer "F.Cu") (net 8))
 (segment (start 198.7 113.5) (end 191.7 113.5) (width 0.508) (layer "F.Cu") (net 8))
 (segment (start 177.1 98.5) (end 170.1 98.5) (width 0.508) (layer "F.Cu") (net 10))
 (segment (start 170.1 98.5) (end 169.4 99.2) (width 0.508) (layer "F.Cu") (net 10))
 (segment (start 129.8 102.5) (end 134.8 102.5) (width 0.508) (layer "F.Cu") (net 9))
 (via (at 129.8 102.5) (size 0.8) (drill 0.4) (layers "F.Cu" "B.Cu") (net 9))
 (via (at 134.8 102.5) (size 0.8) (drill 0.4) (layers "F.Cu" "B.Cu") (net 9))
 (segment (start 164.3 100.5) (end 164.3 98) (width 0.508) (layer "B.Cu") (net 9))
 (segment (start 125.19 102.54) (end 129.76 102.54) (width 0.508) (layer "B.Cu") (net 9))
 (segment (start 129.76 102.54) (end 129.8 102.5) (width 0.508) (layer "B.Cu") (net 9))
 (segment (start 134.8 102.5) (end 162.3 102.5) (width 0.508) (layer "B.Cu") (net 9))
 (segment (start 162.3 102.5) (end 164.3 100.5) (width 0.508) (layer "B.Cu") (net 9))
 (segment (start 127.8 98) (end 128.3 98.5) (width 0.508) (layer "F.Cu") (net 11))
 (segment (start 123.428686 98) (end 127.8 98) (width 0.508) (layer "F.Cu") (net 11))
 (segment (start 131.8 107.5) (end 140.3 107.5) (width 0.508) (layer "F.Cu") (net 11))
 (segment (start 128.3 104) (end 131.8 107.5) (width 0.508) (layer "F.Cu") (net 11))
 (segment (start 122.65 98.778686) (end 123.428686 98) (width 0.508) (layer "F.Cu") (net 11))
 (segment (start 122.65 100) (end 122.65 98.778686) (width 0.508) (layer "F.Cu") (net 11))
 (segment (start 128.3 98.5) (end 128.3 104) (width 0.508) (layer "F.Cu") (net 11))
 (via (at 140.3 107.5) (size 0.8) (drill 0.4) (layers "F.Cu" "B.Cu") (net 11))
 (segment (start 141.8 109) (end 141.8 113) (width 0.508) (layer "B.Cu") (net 11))
 (segment (start 140.3 107.5) (end 141.8 109) (width 0.508) (layer "B.Cu") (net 11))
 (segment (start 155.5 113.5) (end 147.6 113.5) (width 0.508) (layer "F.Cu") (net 12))
 (segment (start 147.6 113.5) (end 146.9 114.2) (width 0.508) (layer "F.Cu") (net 12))
 (segment (start 149.8 98.5) (end 150.3 98) (width 0.508) (layer "F.Cu") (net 14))
 (segment (start 141.9 98.5) (end 149.8 98.5) (width 0.508) (layer "F.Cu") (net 14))
 (segment (start 155.4 102.9) (end 155.4 99.2) (width 0.508) (layer "F.Cu") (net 13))
 (segment (start 152.3 106) (end 155.4 102.9) (width 0.508) (layer "F.Cu") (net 13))
 (via (at 152.3 106) (size 0.8) (drill 0.4) (layers "F.Cu" "B.Cu") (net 13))
 (segment (start 126.11 106) (end 152.3 106) (width 0.508) (layer "B.Cu") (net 13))
 (segment (start 122.65 102.54) (end 126.11 106) (width 0.508) (layer "B.Cu") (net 13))
 (segment (start 111.235899 101.254101) (end 111.235899 106.935899) (width 0.381) (layer "F.Cu") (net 15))
 (segment (start 112.49 100) (end 111.235899 101.254101) (width 0.381) (layer "F.Cu") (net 15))
 (segment (start 111.235899 106.935899) (end 111.3 107) (width 0.381) (layer "F.Cu") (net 15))
 (via (at 111.3 107) (size 0.8) (drill 0.4) (layers "F.Cu" "B.Cu") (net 15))
 (segment (start 133.8 112.5) (end 133.8 114) (width 0.508) (layer "B.Cu") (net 15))
 (segment (start 130.3 109) (end 133.8 112.5) (width 0.508) (layer "B.Cu") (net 15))
 (segment (start 113.3 109) (end 130.3 109) (width 0.508) (layer "B.Cu") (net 15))
 (segment (start 111.3 107) (end 113.3 109) (width 0.508) (layer "B.Cu") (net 15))
 (segment (start 120.3 113.5) (end 128 113.5) (width 0.508) (layer "F.Cu") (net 16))
 (segment (start 128 113.5) (end 128.7 112.8) (width 0.508) (layer "F.Cu") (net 16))
 (segment (start 90.7 98.5) (end 84.6 98.5) (width 0.508) (layer "F.Cu") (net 18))
 (segment (start 84.6 98.5) (end 83.9 99.2) (width 0.508) (layer "F.Cu") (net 18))
 (segment (start 81.3 107) (end 78.8 104.5) (width 0.508) (layer "F.Cu") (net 17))
 (segment (start 78.8 104.5) (end 78.8 98) (width 0.508) (layer "F.Cu") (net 17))
 (via (at 81.3 107) (size 0.8) (drill 0.4) (layers "F.Cu" "B.Cu") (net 17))
 (segment (start 112.49 102.54) (end 112.49 103.761314) (width 0.508) (layer "B.Cu") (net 17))
 (segment (start 109.251314 107) (end 81.3 107) (width 0.508) (layer "B.Cu") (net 17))
 (segment (start 112.49 103.761314) (end 109.251314 107) (width 0.508) (layer "B.Cu") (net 17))
 (segment (start 109.95 100) (end 109.95 98.778686) (width 0.508) (layer "F.Cu") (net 19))
 (segment (start 108.671314 97.5) (end 104.8 97.5) (width 0.508) (layer "F.Cu") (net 19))
 (segment (start 104.8 97.5) (end 101.8 100.5) (width 0.508) (layer "F.Cu") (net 19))
 (segment (start 109.95 98.778686) (end 108.671314 97.5) (width 0.508) (layer "F.Cu") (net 19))
 (segment (start 101.8 108) (end 101.3 108.5) (width 0.508) (layer "F.Cu") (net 19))
 (segment (start 101.8 100.5) (end 101.8 108) (width 0.508) (layer "F.Cu") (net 19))
 (via (at 101.3 108.5) (size 0.8) (drill 0.4) (layers "F.Cu" "B.Cu") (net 19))
 (segment (start 95.8 114) (end 89.8 114) (width 0.508) (layer "B.Cu") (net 19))
 (segment (start 101.3 108.5) (end 95.8 114) (width 0.508) (layer "B.Cu") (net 19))
 (segment (start 84 113.5) (end 84.7 112.8) (width 0.508) (layer "F.Cu") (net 20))
 (segment (start 77.1 113.5) (end 84 113.5) (width 0.508) (layer "F.Cu") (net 20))
 (segment (start 68.9 104.1) (end 68.9 103.9) (width 0.508) (layer "F.Cu") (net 31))
 (segment (start 68.9 103.9) (end 68.9 99.2) (width 0.508) (layer "F.Cu") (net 31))
 (segment (start 70.3 105.5) (end 68.9 104.1) (width 0.508) (layer "F.Cu") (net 31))
 (via (at 70.3 105.5) (size 0.8) (drill 0.4) (layers "F.Cu" "B.Cu") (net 31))
 (segment (start 109.95 102.54) (end 106.99 105.5) (width 0.508) (layer "B.Cu") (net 31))
 (segment (start 106.99 105.5) (end 70.3 105.5) (width 0.508) (layer "B.Cu") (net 31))
 (segment (start 55.5 98.5) (end 63.3 98.5) (width 0.508) (layer "F.Cu") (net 32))
 (segment (start 63.3 98.5) (end 63.8 98) (width 0.508) (layer "F.Cu") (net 32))
 (segment (start 33.9 113.5) (end 42.5 113.5) (width 0.508) (layer "F.Cu") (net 22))
 (segment (start 42.5 113.5) (end 43.2 112.8) (width 0.508) (layer "F.Cu") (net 22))
 (segment (start 97.8 104) (end 97.8 101) (width 0.508) (layer "F.Cu") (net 21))
 (via (at 97.8 104) (size 0.8) (drill 0.4) (layers "F.Cu" "B.Cu") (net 21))
 (via (at 97.8 101) (size 0.8) (drill 0.4) (layers "F.Cu" "B.Cu") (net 21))
 (segment (start 97.8 101) (end 102.8 101) (width 0.508) (layer "B.Cu") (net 21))
 (segment (start 102.8 101) (end 103.8 100) (width 0.508) (layer "B.Cu") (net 21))
 (segment (start 103.8 100) (end 107.41 100) (width 0.508) (layer "B.Cu") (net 21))
 (segment (start 56.878716 104) (end 97.8 104) (width 0.508) (layer "B.Cu") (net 21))
 (segment (start 48.3 114) (end 48.3 112.578716) (width 0.508) (layer "B.Cu") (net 21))
 (segment (start 48.3 112.578716) (end 56.878716 104) (width 0.508) (layer "B.Cu") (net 21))
 (segment (start 41.34 102.54) (end 40.4 101.6) (width 0.508) (layer "B.Cu") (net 23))
 (segment (start 40.4 101.6) (end 40.4 99.2) (width 0.508) (layer "B.Cu") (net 23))
 (segment (start 107.41 102.54) (end 41.34 102.54) (width 0.508) (layer "B.Cu") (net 23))
 (segment (start 26.1 98.5) (end 34.8 98.5) (width 0.508) (layer "F.Cu") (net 24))
 (segment (start 34.8 98.5) (end 35.3 98) (width 0.508) (layer "F.Cu") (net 24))
 (segment (start 259.728489 110.424011) (end 258.365 111.7875) (width 0.254) (layer "B.Cu") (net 33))
 (segment (start 259.728489 105.071511) (end 259.728489 110.424011) (width 0.254) (layer "B.Cu") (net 33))
 (segment (start 260.8 104) (end 259.728489 105.071511) (width 0.254) (layer "B.Cu") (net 33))
 (segment (start 270.9 104) (end 260.8 104) (width 0.254) (layer "B.Cu") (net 33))
 (segment (start 270.63 103) (end 260.3 103) (width 0.254) (layer "B.Cu") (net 34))
 (segment (start 260.3 103) (end 258.365 104.935) (width 0.254) (layer "B.Cu") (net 34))
 (segment (start 258.365 104.935) (end 258.365 109.2475) (width 0.254) (layer "B.Cu") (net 34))
 (segment (start 270.9 102.73) (end 270.63 103) (width 0.254) (layer "B.Cu") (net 34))
 (segment (start 121.300601 105.499399) (end 124.3 108.498798) (width 0.254) (layer "F.Cu") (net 25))
 (segment (start 207.3 111) (end 207.3 112.73) (width 0.254) (layer "F.Cu") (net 25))
 (segment (start 204.798798 108.498798) (end 207.3 111) (width 0.254) (layer "F.Cu") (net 25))
 (segment (start 124.3 108.498798) (end 204.798798 108.498798) (width 0.254) (layer "F.Cu") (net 25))
 (segment (start 120.11 100) (end 121.300601 101.190601) (width 0.254) (layer "F.Cu") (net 25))
 (segment (start 121.300601 101.190601) (end 121.300601 105.499399) (width 0.254) (layer "F.Cu") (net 25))
 (segment (start 203.697817 109.5) (end 123.8 109.5) (width 0.254) (layer "F.Cu") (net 26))
 (segment (start 120.11 105.81) (end 120.11 102.54) (width 0.254) (layer "F.Cu") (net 26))
 (segment (start 205.3 111.102183) (end 203.697817 109.5) (width 0.254) (layer "F.Cu") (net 26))
 (segment (start 205.3 112.754) (end 205.3 111.102183) (width 0.254) (layer "F.Cu") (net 26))
 (segment (start 207.3 114) (end 206.546 114) (width 0.254) (layer "F.Cu") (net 26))
 (segment (start 123.8 109.5) (end 120.11 105.81) (width 0.254) (layer "F.Cu") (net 26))
 (segment (start 206.546 114) (end 205.3 112.754) (width 0.254) (layer "F.Cu") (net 26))
 (segment (start 132.03 97.73) (end 131.3 97) (width 0.254) (layer "B.Cu") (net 27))
 (segment (start 119.3 97) (end 117.57 98.73) (width 0.254) (layer "B.Cu") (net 27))
 (segment (start 133.8 97.73) (end 132.03 97.73) (width 0.254) (layer "B.Cu") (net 27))
 (segment (start 131.3 97) (end 119.3 97) (width 0.254) (layer "B.Cu") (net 27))
 (segment (start 117.57 98.73) (end 117.57 100) (width 0.254) (layer "B.Cu") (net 27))
 (segment (start 131.8 99) (end 133.8 99) (width 0.254) (layer "B.Cu") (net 28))
 (segment (start 130.8 98) (end 131.8 99) (width 0.254) (layer "B.Cu") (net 28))
 (segment (start 118.919399 98.880601) (end 119.8 98) (width 0.254) (layer "B.Cu") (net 28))
 (segment (start 117.57 102.54) (end 118.919399 101.190601) (width 0.254) (layer "B.Cu") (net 28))
 (segment (start 118.919399 101.190601) (end 118.919399 98.880601) (width 0.254) (layer "B.Cu") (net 28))
 (segment (start 119.8 98) (end 130.8 98) (width 0.254) (layer "B.Cu") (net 28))
 (segment (start 93.3 108.5) (end 96.8 112) (width 0.254) (layer "F.Cu") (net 29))
 (segment (start 68.3 112.73) (end 68.3 111) (width 0.254) (layer "F.Cu") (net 29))
 (segment (start 70.8 108.5) (end 93.3 108.5) (width 0.254) (layer "F.Cu") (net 29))
 (segment (start 96.8 112) (end 107.8 112) (width 0.254) (layer "F.Cu") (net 29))
 (segment (start 113.839399 105.960601) (end 113.839399 101.190601) (width 0.254) (layer "F.Cu") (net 29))
 (segment (start 107.8 112) (end 113.839399 105.960601) (width 0.254) (layer "F.Cu") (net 29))
 (segment (start 68.3 111) (end 70.8 108.5) (width 0.254) (layer "F.Cu") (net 29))
 (segment (start 113.839399 101.190601) (end 115.03 100) (width 0.254) (layer "F.Cu") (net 29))
 (segment (start 69.8 110.5) (end 69.8 113.254) (width 0.254) (layer "F.Cu") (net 30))
 (segment (start 108.3 113) (end 96.8 113) (width 0.254) (layer "F.Cu") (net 30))
 (segment (start 70.8 109.5) (end 69.8 110.5) (width 0.254) (layer "F.Cu") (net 30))
 (segment (start 115.03 106.27) (end 108.3 113) (width 0.254) (layer "F.Cu") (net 30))
 (segment (start 115.03 102.54) (end 115.03 106.27) (width 0.254) (layer "F.Cu") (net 30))
 (segment (start 93.3 109.5) (end 70.8 109.5) (width 0.254) (layer "F.Cu") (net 30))
 (segment (start 69.8 113.254) (end 69.054 114) (width 0.254) (layer "F.Cu") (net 30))
 (segment (start 96.8 113) (end 93.3 109.5) (width 0.254) (layer "F.Cu") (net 30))
 (segment (start 69.054 114) (end 68.3 114) (width 0.254) (layer "F.Cu") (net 30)))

